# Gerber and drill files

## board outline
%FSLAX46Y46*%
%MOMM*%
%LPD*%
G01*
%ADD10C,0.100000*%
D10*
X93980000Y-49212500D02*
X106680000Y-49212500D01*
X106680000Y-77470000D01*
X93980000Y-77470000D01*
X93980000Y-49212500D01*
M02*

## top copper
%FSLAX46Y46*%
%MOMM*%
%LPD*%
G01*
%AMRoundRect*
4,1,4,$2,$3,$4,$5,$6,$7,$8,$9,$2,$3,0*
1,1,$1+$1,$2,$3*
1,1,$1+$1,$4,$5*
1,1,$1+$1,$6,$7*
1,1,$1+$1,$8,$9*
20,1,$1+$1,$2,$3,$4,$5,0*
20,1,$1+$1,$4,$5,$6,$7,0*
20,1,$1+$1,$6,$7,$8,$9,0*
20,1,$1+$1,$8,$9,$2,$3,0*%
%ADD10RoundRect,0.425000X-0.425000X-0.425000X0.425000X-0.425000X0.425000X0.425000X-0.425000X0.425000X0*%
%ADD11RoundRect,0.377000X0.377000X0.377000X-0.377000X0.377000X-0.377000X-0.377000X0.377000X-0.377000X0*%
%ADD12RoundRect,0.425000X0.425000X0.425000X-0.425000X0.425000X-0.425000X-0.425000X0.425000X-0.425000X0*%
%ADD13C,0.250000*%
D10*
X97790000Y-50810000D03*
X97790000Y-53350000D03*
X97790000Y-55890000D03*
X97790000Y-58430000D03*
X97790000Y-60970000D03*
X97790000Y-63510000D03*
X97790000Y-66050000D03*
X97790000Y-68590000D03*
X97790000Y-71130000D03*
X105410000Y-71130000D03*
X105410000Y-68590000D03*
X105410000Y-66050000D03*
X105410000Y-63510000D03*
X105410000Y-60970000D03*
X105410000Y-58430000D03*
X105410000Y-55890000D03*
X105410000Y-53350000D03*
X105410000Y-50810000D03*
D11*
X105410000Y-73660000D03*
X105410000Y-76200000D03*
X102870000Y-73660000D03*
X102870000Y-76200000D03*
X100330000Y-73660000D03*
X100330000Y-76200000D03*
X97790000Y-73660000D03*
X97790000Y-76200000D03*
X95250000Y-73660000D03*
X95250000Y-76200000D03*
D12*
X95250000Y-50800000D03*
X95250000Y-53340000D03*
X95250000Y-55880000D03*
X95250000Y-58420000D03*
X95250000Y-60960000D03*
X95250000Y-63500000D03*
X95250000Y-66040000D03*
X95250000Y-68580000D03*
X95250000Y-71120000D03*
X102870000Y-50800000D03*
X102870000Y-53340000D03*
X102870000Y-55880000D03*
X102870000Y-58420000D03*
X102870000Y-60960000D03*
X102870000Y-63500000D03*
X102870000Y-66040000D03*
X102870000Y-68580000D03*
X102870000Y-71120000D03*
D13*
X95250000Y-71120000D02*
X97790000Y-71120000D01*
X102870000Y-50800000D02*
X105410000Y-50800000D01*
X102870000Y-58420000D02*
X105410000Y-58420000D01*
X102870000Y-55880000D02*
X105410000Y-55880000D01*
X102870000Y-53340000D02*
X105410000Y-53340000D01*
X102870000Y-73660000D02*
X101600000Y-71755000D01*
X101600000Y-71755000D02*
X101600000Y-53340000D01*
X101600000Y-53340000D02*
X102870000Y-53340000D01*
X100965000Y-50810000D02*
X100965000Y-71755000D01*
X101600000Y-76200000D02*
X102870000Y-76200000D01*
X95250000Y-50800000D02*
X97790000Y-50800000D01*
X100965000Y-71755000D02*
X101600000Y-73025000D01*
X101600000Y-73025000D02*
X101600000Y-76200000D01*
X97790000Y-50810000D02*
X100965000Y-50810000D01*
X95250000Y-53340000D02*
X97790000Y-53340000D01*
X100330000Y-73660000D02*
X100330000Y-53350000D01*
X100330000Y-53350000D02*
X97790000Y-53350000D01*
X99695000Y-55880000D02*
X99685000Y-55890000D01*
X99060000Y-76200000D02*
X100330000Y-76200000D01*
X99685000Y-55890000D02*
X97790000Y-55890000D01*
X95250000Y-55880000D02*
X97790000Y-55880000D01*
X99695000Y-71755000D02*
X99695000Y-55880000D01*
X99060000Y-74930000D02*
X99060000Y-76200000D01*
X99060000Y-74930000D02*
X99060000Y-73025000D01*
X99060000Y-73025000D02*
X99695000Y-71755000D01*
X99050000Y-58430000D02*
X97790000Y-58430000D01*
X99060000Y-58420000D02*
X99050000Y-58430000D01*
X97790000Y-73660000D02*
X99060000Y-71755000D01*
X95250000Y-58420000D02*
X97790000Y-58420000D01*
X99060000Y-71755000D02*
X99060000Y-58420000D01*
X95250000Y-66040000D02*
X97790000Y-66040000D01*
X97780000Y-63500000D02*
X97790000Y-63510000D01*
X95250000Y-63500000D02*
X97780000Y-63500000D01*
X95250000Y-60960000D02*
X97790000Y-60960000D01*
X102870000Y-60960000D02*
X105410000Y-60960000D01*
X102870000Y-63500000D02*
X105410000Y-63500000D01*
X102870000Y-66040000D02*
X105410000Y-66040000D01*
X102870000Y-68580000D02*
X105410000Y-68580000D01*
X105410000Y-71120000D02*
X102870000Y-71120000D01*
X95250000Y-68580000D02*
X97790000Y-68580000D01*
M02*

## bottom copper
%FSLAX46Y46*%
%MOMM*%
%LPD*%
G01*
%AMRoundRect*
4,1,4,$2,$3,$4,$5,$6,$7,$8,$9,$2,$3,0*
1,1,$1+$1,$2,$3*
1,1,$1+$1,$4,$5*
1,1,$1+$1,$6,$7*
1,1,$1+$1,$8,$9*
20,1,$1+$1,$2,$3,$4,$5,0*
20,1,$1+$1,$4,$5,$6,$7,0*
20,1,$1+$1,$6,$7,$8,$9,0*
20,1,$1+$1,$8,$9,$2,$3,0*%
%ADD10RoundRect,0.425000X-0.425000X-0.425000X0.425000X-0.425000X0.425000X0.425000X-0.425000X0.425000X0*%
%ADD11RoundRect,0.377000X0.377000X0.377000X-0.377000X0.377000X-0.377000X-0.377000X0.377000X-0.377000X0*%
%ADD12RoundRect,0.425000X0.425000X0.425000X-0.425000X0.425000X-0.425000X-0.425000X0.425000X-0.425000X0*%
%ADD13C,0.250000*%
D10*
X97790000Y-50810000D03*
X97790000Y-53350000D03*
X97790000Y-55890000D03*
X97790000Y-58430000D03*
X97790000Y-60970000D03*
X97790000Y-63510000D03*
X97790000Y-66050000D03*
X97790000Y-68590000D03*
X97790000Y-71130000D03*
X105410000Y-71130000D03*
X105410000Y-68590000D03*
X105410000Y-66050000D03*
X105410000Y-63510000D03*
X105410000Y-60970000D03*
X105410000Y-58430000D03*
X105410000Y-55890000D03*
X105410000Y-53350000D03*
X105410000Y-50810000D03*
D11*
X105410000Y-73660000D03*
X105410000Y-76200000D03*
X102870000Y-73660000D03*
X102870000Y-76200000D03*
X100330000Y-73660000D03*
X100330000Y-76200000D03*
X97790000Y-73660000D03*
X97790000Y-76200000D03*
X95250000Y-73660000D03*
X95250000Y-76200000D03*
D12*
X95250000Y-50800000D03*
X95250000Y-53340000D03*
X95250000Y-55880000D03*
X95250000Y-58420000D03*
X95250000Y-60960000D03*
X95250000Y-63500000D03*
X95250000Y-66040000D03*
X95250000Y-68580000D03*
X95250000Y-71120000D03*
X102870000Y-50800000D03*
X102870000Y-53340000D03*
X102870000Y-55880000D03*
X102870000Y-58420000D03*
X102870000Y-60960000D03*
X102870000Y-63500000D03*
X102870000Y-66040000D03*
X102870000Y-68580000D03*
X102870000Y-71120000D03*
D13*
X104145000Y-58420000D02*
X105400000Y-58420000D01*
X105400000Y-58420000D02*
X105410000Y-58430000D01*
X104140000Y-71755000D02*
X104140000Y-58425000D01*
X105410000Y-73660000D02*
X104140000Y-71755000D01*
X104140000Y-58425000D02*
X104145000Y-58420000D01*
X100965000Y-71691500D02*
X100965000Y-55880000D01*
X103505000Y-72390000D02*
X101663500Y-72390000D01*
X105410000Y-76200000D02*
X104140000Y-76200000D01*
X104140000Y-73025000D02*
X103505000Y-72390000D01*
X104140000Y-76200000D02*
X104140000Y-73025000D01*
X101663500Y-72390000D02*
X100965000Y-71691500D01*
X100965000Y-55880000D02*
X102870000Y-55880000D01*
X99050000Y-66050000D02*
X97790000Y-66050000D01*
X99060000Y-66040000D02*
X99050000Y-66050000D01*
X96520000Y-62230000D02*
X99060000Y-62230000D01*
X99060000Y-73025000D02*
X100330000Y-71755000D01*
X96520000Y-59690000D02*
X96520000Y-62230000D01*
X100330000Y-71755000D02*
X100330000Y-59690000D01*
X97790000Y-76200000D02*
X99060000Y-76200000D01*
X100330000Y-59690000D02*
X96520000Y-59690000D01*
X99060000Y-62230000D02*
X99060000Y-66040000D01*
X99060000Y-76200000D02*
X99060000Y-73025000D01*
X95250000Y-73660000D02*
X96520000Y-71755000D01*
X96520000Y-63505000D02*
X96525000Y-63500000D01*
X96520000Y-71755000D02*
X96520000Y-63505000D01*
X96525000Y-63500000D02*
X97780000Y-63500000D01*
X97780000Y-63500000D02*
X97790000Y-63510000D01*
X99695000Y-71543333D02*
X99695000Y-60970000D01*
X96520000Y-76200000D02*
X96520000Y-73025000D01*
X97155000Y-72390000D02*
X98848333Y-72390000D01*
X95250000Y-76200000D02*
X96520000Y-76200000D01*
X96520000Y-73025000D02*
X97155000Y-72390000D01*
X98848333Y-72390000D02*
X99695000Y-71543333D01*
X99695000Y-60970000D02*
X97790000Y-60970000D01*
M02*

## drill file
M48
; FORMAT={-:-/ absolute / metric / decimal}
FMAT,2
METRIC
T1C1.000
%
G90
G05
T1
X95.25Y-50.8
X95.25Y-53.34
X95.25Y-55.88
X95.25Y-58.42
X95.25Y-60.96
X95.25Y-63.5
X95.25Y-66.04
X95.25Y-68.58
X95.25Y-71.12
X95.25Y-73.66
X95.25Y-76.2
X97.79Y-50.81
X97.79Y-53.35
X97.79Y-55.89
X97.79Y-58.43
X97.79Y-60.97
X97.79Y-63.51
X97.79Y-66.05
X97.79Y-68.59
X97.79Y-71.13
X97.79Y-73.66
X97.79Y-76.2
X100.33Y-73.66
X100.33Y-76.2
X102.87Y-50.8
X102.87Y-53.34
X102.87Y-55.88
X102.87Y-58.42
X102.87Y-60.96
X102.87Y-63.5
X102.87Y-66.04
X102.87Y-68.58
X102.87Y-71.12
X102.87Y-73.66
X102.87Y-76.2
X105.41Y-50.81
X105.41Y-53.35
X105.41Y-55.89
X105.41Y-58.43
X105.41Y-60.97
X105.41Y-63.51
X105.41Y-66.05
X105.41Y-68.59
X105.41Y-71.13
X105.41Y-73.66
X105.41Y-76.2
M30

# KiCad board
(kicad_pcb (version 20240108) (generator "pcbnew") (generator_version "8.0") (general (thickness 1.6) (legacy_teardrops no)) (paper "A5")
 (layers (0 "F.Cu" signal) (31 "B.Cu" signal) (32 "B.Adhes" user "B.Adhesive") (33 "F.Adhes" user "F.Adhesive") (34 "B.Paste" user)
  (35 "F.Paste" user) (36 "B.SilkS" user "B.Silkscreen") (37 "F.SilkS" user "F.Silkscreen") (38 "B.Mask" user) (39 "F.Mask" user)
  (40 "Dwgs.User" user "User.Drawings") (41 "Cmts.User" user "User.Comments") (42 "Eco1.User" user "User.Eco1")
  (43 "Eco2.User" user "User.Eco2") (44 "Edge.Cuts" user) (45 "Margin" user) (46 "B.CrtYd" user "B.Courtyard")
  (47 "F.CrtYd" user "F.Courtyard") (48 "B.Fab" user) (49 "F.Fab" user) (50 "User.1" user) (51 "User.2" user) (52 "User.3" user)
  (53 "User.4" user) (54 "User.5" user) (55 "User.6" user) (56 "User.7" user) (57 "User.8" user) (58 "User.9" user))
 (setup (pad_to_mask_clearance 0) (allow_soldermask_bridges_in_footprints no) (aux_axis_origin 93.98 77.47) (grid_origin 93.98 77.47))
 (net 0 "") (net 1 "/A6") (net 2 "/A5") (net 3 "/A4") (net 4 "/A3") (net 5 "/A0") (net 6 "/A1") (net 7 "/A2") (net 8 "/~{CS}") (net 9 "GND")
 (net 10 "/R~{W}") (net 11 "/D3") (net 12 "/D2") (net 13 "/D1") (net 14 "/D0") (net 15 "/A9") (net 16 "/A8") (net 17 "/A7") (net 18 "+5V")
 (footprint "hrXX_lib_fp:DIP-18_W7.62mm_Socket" (layer "F.Cu") (at 97.79 50.81)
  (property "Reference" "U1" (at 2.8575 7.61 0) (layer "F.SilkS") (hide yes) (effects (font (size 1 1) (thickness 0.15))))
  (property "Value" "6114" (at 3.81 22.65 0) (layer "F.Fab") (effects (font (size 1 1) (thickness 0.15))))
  (pad "1" thru_hole roundrect (at 0 0) (size 1.7 1.7) (drill 1) (layers "*.Cu" "*.Mask") (remove_unused_layers no) (roundrect_rratio 0.25)
   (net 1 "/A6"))
  (pad "2" thru_hole roundrect (at 0 2.54) (size 1.7 1.7) (drill 1) (layers "*.Cu" "*.Mask") (remove_unused_layers no)
   (roundrect_rratio 0.25) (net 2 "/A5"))
  (pad "3" thru_hole roundrect (at 0 5.08) (size 1.7 1.7) (drill 1) (layers "*.Cu" "*.Mask") (remove_unused_layers no)
   (roundrect_rratio 0.25) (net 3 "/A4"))
  (pad "4" thru_hole roundrect (at 0 7.62) (size 1.7 1.7) (drill 1) (layers "*.Cu" "*.Mask") (remove_unused_layers no)
   (roundrect_rratio 0.25) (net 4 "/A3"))
  (pad "5" thru_hole roundrect (at 0 10.16) (size 1.7 1.7) (drill 1) (layers "*.Cu" "*.Mask") (remove_unused_layers no)
   (roundrect_rratio 0.25) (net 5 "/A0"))
  (pad "6" thru_hole roundrect (at 0 12.7) (size 1.7 1.7) (drill 1) (layers "*.Cu" "*.Mask") (remove_unused_layers no)
   (roundrect_rratio 0.25) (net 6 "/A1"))
  (pad "7" thru_hole roundrect (at 0 15.24) (size 1.7 1.7) (drill 1) (layers "*.Cu" "*.Mask") (remove_unused_layers no)
   (roundrect_rratio 0.25) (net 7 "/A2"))
  (pad "8" thru_hole roundrect (at 0 17.78) (size 1.7 1.7) (drill 1) (layers "*.Cu" "*.Mask") (remove_unused_layers no)
   (roundrect_rratio 0.25) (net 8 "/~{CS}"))
  (pad "9" thru_hole roundrect (at 0 20.32) (size 1.7 1.7) (drill 1) (layers "*.Cu" "*.Mask") (remove_unused_layers no)
   (roundrect_rratio 0.25) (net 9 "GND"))
  (pad "10" thru_hole roundrect (at 7.62 20.32) (size 1.7 1.7) (drill 1) (layers "*.Cu" "*.Mask") (remove_unused_layers no)
   (roundrect_rratio 0.25) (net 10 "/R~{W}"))
  (pad "11" thru_hole roundrect (at 7.62 17.78) (size 1.7 1.7) (drill 1) (layers "*.Cu" "*.Mask") (remove_unused_layers no)
   (roundrect_rratio 0.25) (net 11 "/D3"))
  (pad "12" thru_hole roundrect (at 7.62 15.24) (size 1.7 1.7) (drill 1) (layers "*.Cu" "*.Mask") (remove_unused_layers no)
   (roundrect_rratio 0.25) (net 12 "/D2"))
  (pad "13" thru_hole roundrect (at 7.62 12.7) (size 1.7 1.7) (drill 1) (layers "*.Cu" "*.Mask") (remove_unused_layers no)
   (roundrect_rratio 0.25) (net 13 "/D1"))
  (pad "14" thru_hole roundrect (at 7.62 10.16) (size 1.7 1.7) (drill 1) (layers "*.Cu" "*.Mask") (remove_unused_layers no)
   (roundrect_rratio 0.25) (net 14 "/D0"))
  (pad "15" thru_hole roundrect (at 7.62 7.62) (size 1.7 1.7) (drill 1) (layers "*.Cu" "*.Mask") (remove_unused_layers no)
   (roundrect_rratio 0.25) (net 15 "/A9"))
  (pad "16" thru_hole roundrect (at 7.62 5.08) (size 1.7 1.7) (drill 1) (layers "*.Cu" "*.Mask") (remove_unused_layers no)
   (roundrect_rratio 0.25) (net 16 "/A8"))
  (pad "17" thru_hole roundrect (at 7.62 2.54) (size 1.7 1.7) (drill 1) (layers "*.Cu" "*.Mask") (remove_unused_layers no)
   (roundrect_rratio 0.25) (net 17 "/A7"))
  (pad "18" thru_hole roundrect (at 7.62 0) (size 1.7 1.7) (drill 1) (layers "*.Cu" "*.Mask") (remove_unused_layers no)
   (roundrect_rratio 0.25) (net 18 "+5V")))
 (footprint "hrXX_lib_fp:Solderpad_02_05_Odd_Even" (layer "F.Cu") (at 105.41 73.66 180)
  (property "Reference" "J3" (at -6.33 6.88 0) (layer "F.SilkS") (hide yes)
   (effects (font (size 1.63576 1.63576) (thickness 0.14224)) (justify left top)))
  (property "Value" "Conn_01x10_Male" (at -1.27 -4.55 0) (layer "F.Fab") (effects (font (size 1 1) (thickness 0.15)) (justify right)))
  (pad "1" thru_hole roundrect (at 0 0 180) (size 1.508 1.508) (drill 1) (layers "*.Cu" "*.Mask") (remove_unused_layers no)
   (roundrect_rratio 0.25) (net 15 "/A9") (solder_mask_margin 0.1016))
  (pad "2" thru_hole roundrect (at 0 -2.54 180) (size 1.508 1.508) (drill 1) (layers "*.Cu" "*.Mask") (remove_unused_layers no)
   (roundrect_rratio 0.25) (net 16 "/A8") (solder_mask_margin 0.1016))
  (pad "3" thru_hole roundrect (at 2.54 0 180) (size 1.508 1.508) (drill 1) (layers "*.Cu" "*.Mask") (remove_unused_layers no)
   (roundrect_rratio 0.25) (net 17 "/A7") (solder_mask_margin 0.1016))
  (pad "4" thru_hole roundrect (at 2.54 -2.54 180) (size 1.508 1.508) (drill 1) (layers "*.Cu" "*.Mask") (remove_unused_layers no)
   (roundrect_rratio 0.25) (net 1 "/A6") (solder_mask_margin 0.1016))
  (pad "5" thru_hole roundrect (at 5.08 0 180) (size 1.508 1.508) (drill 1) (layers "*.Cu" "*.Mask") (remove_unused_layers no)
   (roundrect_rratio 0.25) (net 2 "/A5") (solder_mask_margin 0.1016))
  (pad "6" thru_hole roundrect (at 5.08 -2.54 180) (size 1.508 1.508) (drill 1) (layers "*.Cu" "*.Mask") (remove_unused_layers no)
   (roundrect_rratio 0.25) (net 3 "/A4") (solder_mask_margin 0.1016))
  (pad "7" thru_hole roundrect (at 7.62 0 180) (size 1.508 1.508) (drill 1) (layers "*.Cu" "*.Mask") (remove_unused_layers no)
   (roundrect_rratio 0.25) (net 4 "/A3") (solder_mask_margin 0.1016))
  (pad "8" thru_hole roundrect (at 7.62 -2.54 180) (size 1.508 1.508) (drill 1) (layers "*.Cu" "*.Mask") (remove_unused_layers no)
   (roundrect_rratio 0.25) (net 7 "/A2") (solder_mask_margin 0.1016))
  (pad "9" thru_hole roundrect (at 10.16 0 180) (size 1.508 1.508) (drill 1) (layers "*.Cu" "*.Mask") (remove_unused_layers no)
   (roundrect_rratio 0.25) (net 6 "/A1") (solder_mask_margin 0.1016))
  (pad "10" thru_hole roundrect (at 10.16 -2.54 180) (size 1.508 1.508) (drill 1) (layers "*.Cu" "*.Mask") (remove_unused_layers no)
   (roundrect_rratio 0.25) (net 5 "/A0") (solder_mask_margin 0.1016)))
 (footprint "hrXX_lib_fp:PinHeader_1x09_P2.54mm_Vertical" (layer "B.Cu") (at 95.25 50.8 180)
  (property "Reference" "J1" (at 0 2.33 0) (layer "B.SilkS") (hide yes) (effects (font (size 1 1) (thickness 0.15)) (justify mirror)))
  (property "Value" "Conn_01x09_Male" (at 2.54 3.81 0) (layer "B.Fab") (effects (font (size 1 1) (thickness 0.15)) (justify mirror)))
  (pad "1" thru_hole roundrect (at 0 0 180) (size 1.7 1.7) (drill 1) (layers "*.Cu" "*.Mask") (remove_unused_layers no)
   (roundrect_rratio 0.25) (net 1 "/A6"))
  (pad "2" thru_hole roundrect (at 0 -2.54 180) (size 1.7 1.7) (drill 1) (layers "*.Cu" "*.Mask") (remove_unused_layers no)
   (roundrect_rratio 0.25) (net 2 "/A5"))
  (pad "3" thru_hole roundrect (at 0 -5.08 180) (size 1.7 1.7) (drill 1) (layers "*.Cu" "*.Mask") (remove_unused_layers no)
   (roundrect_rratio 0.25) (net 3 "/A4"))
  (pad "4" thru_hole roundrect (at 0 -7.62 180) (size 1.7 1.7) (drill 1) (layers "*.Cu" "*.Mask") (remove_unused_layers no)
   (roundrect_rratio 0.25) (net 4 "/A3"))
  (pad "5" thru_hole roundrect (at 0 -10.16 180) (size 1.7 1.7) (drill 1) (layers "*.Cu" "*.Mask") (remove_unused_layers no)
   (roundrect_rratio 0.25) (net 5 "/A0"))
  (pad "6" thru_hole roundrect (at 0 -12.7 180) (size 1.7 1.7) (drill 1) (layers "*.Cu" "*.Mask") (remove_unused_layers no)
   (roundrect_rratio 0.25) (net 6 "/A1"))
  (pad "7" thru_hole roundrect (at 0 -15.24 180) (size 1.7 1.7) (drill 1) (layers "*.Cu" "*.Mask") (remove_unused_layers no)
   (roundrect_rratio 0.25) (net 7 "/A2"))
  (pad "8" thru_hole roundrect (at 0 -17.78 180) (size 1.7 1.7) (drill 1) (layers "*.Cu" "*.Mask") (remove_unused_layers no)
   (roundrect_rratio 0.25) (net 8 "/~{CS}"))
  (pad "9" thru_hole roundrect (at 0 -20.32 180) (size 1.7 1.7) (drill 1) (layers "*.Cu" "*.Mask") (remove_unused_layers no)
   (roundrect_rratio 0.25) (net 9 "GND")))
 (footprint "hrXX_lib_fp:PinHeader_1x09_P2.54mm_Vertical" (layer "B.Cu") (at 102.87 50.8 180)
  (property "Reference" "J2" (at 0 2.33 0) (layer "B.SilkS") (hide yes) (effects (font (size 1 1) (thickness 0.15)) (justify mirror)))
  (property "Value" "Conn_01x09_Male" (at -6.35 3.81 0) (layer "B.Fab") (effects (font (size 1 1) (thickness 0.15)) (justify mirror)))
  (pad "1" thru_hole roundrect (at 0 0 180) (size 1.7 1.7) (drill 1) (layers "*.Cu" "*.Mask") (remove_unused_layers no)
   (roundrect_rratio 0.25) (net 18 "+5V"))
  (pad "2" thru_hole roundrect (at 0 -2.54 180) (size 1.7 1.7) (drill 1) (layers "*.Cu" "*.Mask") (remove_unused_layers no)
   (roundrect_rratio 0.25) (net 17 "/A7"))
  (pad "3" thru_hole roundrect (at 0 -5.08 180) (size 1.7 1.7) (drill 1) (layers "*.Cu" "*.Mask") (remove_unused_layers no)
   (roundrect_rratio 0.25) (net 16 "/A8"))
  (pad "4" thru_hole roundrect (at 0 -7.62 180) (size 1.7 1.7) (drill 1) (layers "*.Cu" "*.Mask") (remove_unused_layers no)
   (roundrect_rratio 0.25) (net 15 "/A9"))
  (pad "5" thru_hole roundrect (at 0 -10.16 180) (size 1.7 1.7) (drill 1) (layers "*.Cu" "*.Mask") (remove_unused_layers no)
   (roundrect_rratio 0.25) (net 14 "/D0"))
  (pad "6" thru_hole roundrect (at 0 -12.7 180) (size 1.7 1.7) (drill 1) (layers "*.Cu" "*.Mask") (remove_unused_layers no)
   (roundrect_rratio 0.25) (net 13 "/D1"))
  (pad "7" thru_hole roundrect (at 0 -15.24 180) (size 1.7 1.7) (drill 1) (layers "*.Cu" "*.Mask") (remove_unused_layers no)
   (roundrect_rratio 0.25) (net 12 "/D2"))
  (pad "8" thru_hole roundrect (at 0 -17.78 180) (size 1.7 1.7) (drill 1) (layers "*.Cu" "*.Mask") (remove_unused_layers no)
   (roundrect_rratio 0.25) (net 11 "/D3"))
  (pad "9" thru_hole roundrect (at 0 -20.32 180) (size 1.7 1.7) (drill 1) (layers "*.Cu" "*.Mask") (remove_unused_layers no)
   (roundrect_rratio 0.25) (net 10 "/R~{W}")))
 (gr_rect (start 93.98 49.2125) (end 106.68 77.47) (stroke (width 0.1) (type default)) (fill none) (layer "Edge.Cuts"))
 (segment (start 95.25 71.12) (end 97.79 71.12) (width 0.25) (layer "F.Cu") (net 9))
 (segment (start 102.87 50.8) (end 105.41 50.8) (width 0.25) (layer "F.Cu") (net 18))
 (segment (start 102.87 58.42) (end 105.41 58.42) (width 0.25) (layer "F.Cu") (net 15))
 (segment (start 104.145 58.42) (end 105.4 58.42) (width 0.25) (layer "B.Cu") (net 15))
 (segment (start 105.4 58.42) (end 105.41 58.43) (width 0.25) (layer "B.Cu") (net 15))
 (segment (start 104.14 71.755) (end 104.14 58.425) (width 0.25) (layer "B.Cu") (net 15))
 (segment (start 105.41 73.66) (end 104.14 71.755) (width 0.25) (layer "B.Cu") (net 15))
 (segment (start 104.14 58.425) (end 104.145 58.42) (width 0.25) (layer "B.Cu") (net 15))
 (segment (start 102.87 55.88) (end 105.41 55.88) (width 0.25) (layer "F.Cu") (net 16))
 (segment (start 100.965 71.6915) (end 100.965 55.88) (width 0.25) (layer "B.Cu") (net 16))
 (segment (start 103.505 72.39) (end 101.6635 72.39) (width 0.25) (layer "B.Cu") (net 16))
 (segment (start 105.41 76.2) (end 104.14 76.2) (width 0.25) (layer "B.Cu") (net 16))
 (segment (start 104.14 73.025) (end 103.505 72.39) (width 0.25) (layer "B.Cu") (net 16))
 (segment (start 104.14 76.2) (end 104.14 73.025) (width 0.25) (layer "B.Cu") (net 16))
 (segment (start 101.6635 72.39) (end 100.965 71.6915) (width 0.25) (layer "B.Cu") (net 16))
 (segment (start 100.965 55.88) (end 102.87 55.88) (width 0.25) (layer "B.Cu") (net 16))
 (segment (start 102.87 53.34) (end 105.41 53.34) (width 0.25) (layer "F.Cu") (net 17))
 (segment (start 102.87 73.66) (end 101.6 71.755) (width 0.25) (layer "F.Cu") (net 17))
 (segment (start 101.6 71.755) (end 101.6 53.34) (width 0.25) (layer "F.Cu") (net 17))
 (segment (start 101.6 53.34) (end 102.87 53.34) (width 0.25) (layer "F.Cu") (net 17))
 (segment (start 100.965 50.81) (end 100.965 71.755) (width 0.25) (layer "F.Cu") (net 1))
 (segment (start 101.6 76.2) (end 102.87 76.2) (width 0.25) (layer "F.Cu") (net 1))
 (segment (start 95.25 50.8) (end 97.79 50.8) (width 0.25) (layer "F.Cu") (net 1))
 (segment (start 100.965 71.755) (end 101.6 73.025) (width 0.25) (layer "F.Cu") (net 1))
 (segment (start 101.6 73.025) (end 101.6 76.2) (width 0.25) (layer "F.Cu") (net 1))
 (segment (start 97.79 50.81) (end 100.965 50.81) (width 0.25) (layer "F.Cu") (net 1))
 (segment (start 95.25 53.34) (end 97.79 53.34) (width 0.25) (layer "F.Cu") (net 2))
 (segment (start 100.33 73.66) (end 100.33 53.35) (width 0.25) (layer "F.Cu") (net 2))
 (segment (start 100.33 53.35) (end 97.79 53.35) (width 0.25) (layer "F.Cu") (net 2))
 (segment (start 99.695 55.88) (end 99.685 55.89) (width 0.25) (layer "F.Cu") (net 3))
 (segment (start 99.06 76.2) (end 100.33 76.2) (width 0.25) (layer "F.Cu") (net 3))
 (segment (start 99.685 55.89) (end 97.79 55.89) (width 0.25) (layer "F.Cu") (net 3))
 (segment (start 95.25 55.88) (end 97.79 55.88) (width 0.25) (layer "F.Cu") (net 3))
 (segment (start 99.695 71.755) (end 99.695 55.88) (width 0.25) (layer "F.Cu") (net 3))
 (segment (start 99.06 74.93) (end 99.06 76.2) (width 0.25) (layer "F.Cu") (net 3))
 (segment (start 99.06 74.93) (end 99.06 73.025) (width 0.25) (layer "F.Cu") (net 3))
 (segment (start 99.06 73.025) (end 99.695 71.755) (width 0.25) (layer "F.Cu") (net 3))
 (segment (start 99.05 58.43) (end 97.79 58.43) (width 0.25) (layer "F.Cu") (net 4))
 (segment (start 99.06 58.42) (end 99.05 58.43) (width 0.25) (layer "F.Cu") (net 4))
 (segment (start 97.79 73.66) (end 99.06 71.755) (width 0.25) (layer "F.Cu") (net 4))
 (segment (start 95.25 58.42) (end 97.79 58.42) (width 0.25) (layer "F.Cu") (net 4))
 (segment (start 99.06 71.755) (end 99.06 58.42) (width 0.25) (layer "F.Cu") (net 4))
 (segment (start 95.25 66.04) (end 97.79 66.04) (width 0.25) (layer "F.Cu") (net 7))
 (segment (start 99.05 66.05) (end 97.79 66.05) (width 0.25) (layer "B.Cu") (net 7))
 (segment (start 99.06 66.04) (end 99.05 66.05) (width 0.25) (layer "B.Cu") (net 7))
 (segment (start 96.52 62.23) (end 99.06 62.23) (width 0.25) (layer "B.Cu") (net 7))
 (segment (start 99.06 73.025) (end 100.33 71.755) (width 0.25) (layer "B.Cu") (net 7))
 (segment (start 96.52 59.69) (end 96.52 62.23) (width 0.25) (layer "B.Cu") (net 7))
 (segment (start 100.33 71.755) (end 100.33 59.69) (width 0.25) (layer "B.Cu") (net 7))
 (segment (start 97.79 76.2) (end 99.06 76.2) (width 0.25) (layer "B.Cu") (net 7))
 (segment (start 100.33 59.69) (end 96.52 59.69) (width 0.25) (layer "B.Cu") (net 7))
 (segment (start 99.06 62.23) (end 99.06 66.04) (width 0.25) (layer "B.Cu") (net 7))
 (segment (start 99.06 76.2) (end 99.06 73.025) (width 0.25) (layer "B.Cu") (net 7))
 (segment (start 97.78 63.5) (end 97.79 63.51) (width 0.25) (layer "F.Cu") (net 6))
 (segment (start 95.25 63.5) (end 97.78 63.5) (width 0.25) (layer "F.Cu") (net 6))
 (segment (start 95.25 73.66) (end 96.52 71.755) (width 0.25) (layer "B.Cu") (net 6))
 (segment (start 96.52 63.505) (end 96.525 63.5) (width 0.25) (layer "B.Cu") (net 6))
 (segment (start 96.52 71.755) (end 96.52 63.505) (width 0.25) (layer "B.Cu") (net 6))
 (segment (start 96.525 63.5) (end 97.78 63.5) (width 0.25) (layer "B.Cu") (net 6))
 (segment (start 97.78 63.5) (end 97.79 63.51) (width 0.25) (layer "B.Cu") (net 6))
 (segment (start 95.25 60.96) (end 97.79 60.96) (width 0.25) (layer "F.Cu") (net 5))
 (segment (start 99.695 71.543333) (end 99.695 60.97) (width 0.25) (layer "B.Cu") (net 5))
 (segment (start 96.52 76.2) (end 96.52 73.025) (width 0.25) (layer "B.Cu") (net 5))
 (segment (start 97.155 72.39) (end 98.848333 72.39) (width 0.25) (layer "B.Cu") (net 5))
 (segment (start 95.25 76.2) (end 96.52 76.2) (width 0.25) (layer "B.Cu") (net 5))
 (segment (start 96.52 73.025) (end 97.155 72.39) (width 0.25) (layer "B.Cu") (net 5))
 (segment (start 98.848333 72.39) (end 99.695 71.543333) (width 0.25) (layer "B.Cu") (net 5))
 (segment (start 99.695 60.97) (end 97.79 60.97) (width 0.25) (layer "B.Cu") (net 5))
 (segment (start 102.87 60.96) (end 105.41 60.96) (width 0.25) (layer "F.Cu") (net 14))
 (segment (start 102.87 63.5) (end 105.41 63.5) (width 0.25) (layer "F.Cu") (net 13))
 (segment (start 102.87 66.04) (end 105.41 66.04) (width 0.25) (layer "F.Cu") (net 12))
 (segment (start 102.87 68.58) (end 105.41 68.58) (width 0.25) (layer "F.Cu") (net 11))
 (segment (start 105.41 71.12) (end 102.87 71.12) (width 0.25) (layer "F.Cu") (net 10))
 (segment (start 95.25 68.58) (end 97.79 68.58) (width 0.25) (layer "F.Cu") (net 8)))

